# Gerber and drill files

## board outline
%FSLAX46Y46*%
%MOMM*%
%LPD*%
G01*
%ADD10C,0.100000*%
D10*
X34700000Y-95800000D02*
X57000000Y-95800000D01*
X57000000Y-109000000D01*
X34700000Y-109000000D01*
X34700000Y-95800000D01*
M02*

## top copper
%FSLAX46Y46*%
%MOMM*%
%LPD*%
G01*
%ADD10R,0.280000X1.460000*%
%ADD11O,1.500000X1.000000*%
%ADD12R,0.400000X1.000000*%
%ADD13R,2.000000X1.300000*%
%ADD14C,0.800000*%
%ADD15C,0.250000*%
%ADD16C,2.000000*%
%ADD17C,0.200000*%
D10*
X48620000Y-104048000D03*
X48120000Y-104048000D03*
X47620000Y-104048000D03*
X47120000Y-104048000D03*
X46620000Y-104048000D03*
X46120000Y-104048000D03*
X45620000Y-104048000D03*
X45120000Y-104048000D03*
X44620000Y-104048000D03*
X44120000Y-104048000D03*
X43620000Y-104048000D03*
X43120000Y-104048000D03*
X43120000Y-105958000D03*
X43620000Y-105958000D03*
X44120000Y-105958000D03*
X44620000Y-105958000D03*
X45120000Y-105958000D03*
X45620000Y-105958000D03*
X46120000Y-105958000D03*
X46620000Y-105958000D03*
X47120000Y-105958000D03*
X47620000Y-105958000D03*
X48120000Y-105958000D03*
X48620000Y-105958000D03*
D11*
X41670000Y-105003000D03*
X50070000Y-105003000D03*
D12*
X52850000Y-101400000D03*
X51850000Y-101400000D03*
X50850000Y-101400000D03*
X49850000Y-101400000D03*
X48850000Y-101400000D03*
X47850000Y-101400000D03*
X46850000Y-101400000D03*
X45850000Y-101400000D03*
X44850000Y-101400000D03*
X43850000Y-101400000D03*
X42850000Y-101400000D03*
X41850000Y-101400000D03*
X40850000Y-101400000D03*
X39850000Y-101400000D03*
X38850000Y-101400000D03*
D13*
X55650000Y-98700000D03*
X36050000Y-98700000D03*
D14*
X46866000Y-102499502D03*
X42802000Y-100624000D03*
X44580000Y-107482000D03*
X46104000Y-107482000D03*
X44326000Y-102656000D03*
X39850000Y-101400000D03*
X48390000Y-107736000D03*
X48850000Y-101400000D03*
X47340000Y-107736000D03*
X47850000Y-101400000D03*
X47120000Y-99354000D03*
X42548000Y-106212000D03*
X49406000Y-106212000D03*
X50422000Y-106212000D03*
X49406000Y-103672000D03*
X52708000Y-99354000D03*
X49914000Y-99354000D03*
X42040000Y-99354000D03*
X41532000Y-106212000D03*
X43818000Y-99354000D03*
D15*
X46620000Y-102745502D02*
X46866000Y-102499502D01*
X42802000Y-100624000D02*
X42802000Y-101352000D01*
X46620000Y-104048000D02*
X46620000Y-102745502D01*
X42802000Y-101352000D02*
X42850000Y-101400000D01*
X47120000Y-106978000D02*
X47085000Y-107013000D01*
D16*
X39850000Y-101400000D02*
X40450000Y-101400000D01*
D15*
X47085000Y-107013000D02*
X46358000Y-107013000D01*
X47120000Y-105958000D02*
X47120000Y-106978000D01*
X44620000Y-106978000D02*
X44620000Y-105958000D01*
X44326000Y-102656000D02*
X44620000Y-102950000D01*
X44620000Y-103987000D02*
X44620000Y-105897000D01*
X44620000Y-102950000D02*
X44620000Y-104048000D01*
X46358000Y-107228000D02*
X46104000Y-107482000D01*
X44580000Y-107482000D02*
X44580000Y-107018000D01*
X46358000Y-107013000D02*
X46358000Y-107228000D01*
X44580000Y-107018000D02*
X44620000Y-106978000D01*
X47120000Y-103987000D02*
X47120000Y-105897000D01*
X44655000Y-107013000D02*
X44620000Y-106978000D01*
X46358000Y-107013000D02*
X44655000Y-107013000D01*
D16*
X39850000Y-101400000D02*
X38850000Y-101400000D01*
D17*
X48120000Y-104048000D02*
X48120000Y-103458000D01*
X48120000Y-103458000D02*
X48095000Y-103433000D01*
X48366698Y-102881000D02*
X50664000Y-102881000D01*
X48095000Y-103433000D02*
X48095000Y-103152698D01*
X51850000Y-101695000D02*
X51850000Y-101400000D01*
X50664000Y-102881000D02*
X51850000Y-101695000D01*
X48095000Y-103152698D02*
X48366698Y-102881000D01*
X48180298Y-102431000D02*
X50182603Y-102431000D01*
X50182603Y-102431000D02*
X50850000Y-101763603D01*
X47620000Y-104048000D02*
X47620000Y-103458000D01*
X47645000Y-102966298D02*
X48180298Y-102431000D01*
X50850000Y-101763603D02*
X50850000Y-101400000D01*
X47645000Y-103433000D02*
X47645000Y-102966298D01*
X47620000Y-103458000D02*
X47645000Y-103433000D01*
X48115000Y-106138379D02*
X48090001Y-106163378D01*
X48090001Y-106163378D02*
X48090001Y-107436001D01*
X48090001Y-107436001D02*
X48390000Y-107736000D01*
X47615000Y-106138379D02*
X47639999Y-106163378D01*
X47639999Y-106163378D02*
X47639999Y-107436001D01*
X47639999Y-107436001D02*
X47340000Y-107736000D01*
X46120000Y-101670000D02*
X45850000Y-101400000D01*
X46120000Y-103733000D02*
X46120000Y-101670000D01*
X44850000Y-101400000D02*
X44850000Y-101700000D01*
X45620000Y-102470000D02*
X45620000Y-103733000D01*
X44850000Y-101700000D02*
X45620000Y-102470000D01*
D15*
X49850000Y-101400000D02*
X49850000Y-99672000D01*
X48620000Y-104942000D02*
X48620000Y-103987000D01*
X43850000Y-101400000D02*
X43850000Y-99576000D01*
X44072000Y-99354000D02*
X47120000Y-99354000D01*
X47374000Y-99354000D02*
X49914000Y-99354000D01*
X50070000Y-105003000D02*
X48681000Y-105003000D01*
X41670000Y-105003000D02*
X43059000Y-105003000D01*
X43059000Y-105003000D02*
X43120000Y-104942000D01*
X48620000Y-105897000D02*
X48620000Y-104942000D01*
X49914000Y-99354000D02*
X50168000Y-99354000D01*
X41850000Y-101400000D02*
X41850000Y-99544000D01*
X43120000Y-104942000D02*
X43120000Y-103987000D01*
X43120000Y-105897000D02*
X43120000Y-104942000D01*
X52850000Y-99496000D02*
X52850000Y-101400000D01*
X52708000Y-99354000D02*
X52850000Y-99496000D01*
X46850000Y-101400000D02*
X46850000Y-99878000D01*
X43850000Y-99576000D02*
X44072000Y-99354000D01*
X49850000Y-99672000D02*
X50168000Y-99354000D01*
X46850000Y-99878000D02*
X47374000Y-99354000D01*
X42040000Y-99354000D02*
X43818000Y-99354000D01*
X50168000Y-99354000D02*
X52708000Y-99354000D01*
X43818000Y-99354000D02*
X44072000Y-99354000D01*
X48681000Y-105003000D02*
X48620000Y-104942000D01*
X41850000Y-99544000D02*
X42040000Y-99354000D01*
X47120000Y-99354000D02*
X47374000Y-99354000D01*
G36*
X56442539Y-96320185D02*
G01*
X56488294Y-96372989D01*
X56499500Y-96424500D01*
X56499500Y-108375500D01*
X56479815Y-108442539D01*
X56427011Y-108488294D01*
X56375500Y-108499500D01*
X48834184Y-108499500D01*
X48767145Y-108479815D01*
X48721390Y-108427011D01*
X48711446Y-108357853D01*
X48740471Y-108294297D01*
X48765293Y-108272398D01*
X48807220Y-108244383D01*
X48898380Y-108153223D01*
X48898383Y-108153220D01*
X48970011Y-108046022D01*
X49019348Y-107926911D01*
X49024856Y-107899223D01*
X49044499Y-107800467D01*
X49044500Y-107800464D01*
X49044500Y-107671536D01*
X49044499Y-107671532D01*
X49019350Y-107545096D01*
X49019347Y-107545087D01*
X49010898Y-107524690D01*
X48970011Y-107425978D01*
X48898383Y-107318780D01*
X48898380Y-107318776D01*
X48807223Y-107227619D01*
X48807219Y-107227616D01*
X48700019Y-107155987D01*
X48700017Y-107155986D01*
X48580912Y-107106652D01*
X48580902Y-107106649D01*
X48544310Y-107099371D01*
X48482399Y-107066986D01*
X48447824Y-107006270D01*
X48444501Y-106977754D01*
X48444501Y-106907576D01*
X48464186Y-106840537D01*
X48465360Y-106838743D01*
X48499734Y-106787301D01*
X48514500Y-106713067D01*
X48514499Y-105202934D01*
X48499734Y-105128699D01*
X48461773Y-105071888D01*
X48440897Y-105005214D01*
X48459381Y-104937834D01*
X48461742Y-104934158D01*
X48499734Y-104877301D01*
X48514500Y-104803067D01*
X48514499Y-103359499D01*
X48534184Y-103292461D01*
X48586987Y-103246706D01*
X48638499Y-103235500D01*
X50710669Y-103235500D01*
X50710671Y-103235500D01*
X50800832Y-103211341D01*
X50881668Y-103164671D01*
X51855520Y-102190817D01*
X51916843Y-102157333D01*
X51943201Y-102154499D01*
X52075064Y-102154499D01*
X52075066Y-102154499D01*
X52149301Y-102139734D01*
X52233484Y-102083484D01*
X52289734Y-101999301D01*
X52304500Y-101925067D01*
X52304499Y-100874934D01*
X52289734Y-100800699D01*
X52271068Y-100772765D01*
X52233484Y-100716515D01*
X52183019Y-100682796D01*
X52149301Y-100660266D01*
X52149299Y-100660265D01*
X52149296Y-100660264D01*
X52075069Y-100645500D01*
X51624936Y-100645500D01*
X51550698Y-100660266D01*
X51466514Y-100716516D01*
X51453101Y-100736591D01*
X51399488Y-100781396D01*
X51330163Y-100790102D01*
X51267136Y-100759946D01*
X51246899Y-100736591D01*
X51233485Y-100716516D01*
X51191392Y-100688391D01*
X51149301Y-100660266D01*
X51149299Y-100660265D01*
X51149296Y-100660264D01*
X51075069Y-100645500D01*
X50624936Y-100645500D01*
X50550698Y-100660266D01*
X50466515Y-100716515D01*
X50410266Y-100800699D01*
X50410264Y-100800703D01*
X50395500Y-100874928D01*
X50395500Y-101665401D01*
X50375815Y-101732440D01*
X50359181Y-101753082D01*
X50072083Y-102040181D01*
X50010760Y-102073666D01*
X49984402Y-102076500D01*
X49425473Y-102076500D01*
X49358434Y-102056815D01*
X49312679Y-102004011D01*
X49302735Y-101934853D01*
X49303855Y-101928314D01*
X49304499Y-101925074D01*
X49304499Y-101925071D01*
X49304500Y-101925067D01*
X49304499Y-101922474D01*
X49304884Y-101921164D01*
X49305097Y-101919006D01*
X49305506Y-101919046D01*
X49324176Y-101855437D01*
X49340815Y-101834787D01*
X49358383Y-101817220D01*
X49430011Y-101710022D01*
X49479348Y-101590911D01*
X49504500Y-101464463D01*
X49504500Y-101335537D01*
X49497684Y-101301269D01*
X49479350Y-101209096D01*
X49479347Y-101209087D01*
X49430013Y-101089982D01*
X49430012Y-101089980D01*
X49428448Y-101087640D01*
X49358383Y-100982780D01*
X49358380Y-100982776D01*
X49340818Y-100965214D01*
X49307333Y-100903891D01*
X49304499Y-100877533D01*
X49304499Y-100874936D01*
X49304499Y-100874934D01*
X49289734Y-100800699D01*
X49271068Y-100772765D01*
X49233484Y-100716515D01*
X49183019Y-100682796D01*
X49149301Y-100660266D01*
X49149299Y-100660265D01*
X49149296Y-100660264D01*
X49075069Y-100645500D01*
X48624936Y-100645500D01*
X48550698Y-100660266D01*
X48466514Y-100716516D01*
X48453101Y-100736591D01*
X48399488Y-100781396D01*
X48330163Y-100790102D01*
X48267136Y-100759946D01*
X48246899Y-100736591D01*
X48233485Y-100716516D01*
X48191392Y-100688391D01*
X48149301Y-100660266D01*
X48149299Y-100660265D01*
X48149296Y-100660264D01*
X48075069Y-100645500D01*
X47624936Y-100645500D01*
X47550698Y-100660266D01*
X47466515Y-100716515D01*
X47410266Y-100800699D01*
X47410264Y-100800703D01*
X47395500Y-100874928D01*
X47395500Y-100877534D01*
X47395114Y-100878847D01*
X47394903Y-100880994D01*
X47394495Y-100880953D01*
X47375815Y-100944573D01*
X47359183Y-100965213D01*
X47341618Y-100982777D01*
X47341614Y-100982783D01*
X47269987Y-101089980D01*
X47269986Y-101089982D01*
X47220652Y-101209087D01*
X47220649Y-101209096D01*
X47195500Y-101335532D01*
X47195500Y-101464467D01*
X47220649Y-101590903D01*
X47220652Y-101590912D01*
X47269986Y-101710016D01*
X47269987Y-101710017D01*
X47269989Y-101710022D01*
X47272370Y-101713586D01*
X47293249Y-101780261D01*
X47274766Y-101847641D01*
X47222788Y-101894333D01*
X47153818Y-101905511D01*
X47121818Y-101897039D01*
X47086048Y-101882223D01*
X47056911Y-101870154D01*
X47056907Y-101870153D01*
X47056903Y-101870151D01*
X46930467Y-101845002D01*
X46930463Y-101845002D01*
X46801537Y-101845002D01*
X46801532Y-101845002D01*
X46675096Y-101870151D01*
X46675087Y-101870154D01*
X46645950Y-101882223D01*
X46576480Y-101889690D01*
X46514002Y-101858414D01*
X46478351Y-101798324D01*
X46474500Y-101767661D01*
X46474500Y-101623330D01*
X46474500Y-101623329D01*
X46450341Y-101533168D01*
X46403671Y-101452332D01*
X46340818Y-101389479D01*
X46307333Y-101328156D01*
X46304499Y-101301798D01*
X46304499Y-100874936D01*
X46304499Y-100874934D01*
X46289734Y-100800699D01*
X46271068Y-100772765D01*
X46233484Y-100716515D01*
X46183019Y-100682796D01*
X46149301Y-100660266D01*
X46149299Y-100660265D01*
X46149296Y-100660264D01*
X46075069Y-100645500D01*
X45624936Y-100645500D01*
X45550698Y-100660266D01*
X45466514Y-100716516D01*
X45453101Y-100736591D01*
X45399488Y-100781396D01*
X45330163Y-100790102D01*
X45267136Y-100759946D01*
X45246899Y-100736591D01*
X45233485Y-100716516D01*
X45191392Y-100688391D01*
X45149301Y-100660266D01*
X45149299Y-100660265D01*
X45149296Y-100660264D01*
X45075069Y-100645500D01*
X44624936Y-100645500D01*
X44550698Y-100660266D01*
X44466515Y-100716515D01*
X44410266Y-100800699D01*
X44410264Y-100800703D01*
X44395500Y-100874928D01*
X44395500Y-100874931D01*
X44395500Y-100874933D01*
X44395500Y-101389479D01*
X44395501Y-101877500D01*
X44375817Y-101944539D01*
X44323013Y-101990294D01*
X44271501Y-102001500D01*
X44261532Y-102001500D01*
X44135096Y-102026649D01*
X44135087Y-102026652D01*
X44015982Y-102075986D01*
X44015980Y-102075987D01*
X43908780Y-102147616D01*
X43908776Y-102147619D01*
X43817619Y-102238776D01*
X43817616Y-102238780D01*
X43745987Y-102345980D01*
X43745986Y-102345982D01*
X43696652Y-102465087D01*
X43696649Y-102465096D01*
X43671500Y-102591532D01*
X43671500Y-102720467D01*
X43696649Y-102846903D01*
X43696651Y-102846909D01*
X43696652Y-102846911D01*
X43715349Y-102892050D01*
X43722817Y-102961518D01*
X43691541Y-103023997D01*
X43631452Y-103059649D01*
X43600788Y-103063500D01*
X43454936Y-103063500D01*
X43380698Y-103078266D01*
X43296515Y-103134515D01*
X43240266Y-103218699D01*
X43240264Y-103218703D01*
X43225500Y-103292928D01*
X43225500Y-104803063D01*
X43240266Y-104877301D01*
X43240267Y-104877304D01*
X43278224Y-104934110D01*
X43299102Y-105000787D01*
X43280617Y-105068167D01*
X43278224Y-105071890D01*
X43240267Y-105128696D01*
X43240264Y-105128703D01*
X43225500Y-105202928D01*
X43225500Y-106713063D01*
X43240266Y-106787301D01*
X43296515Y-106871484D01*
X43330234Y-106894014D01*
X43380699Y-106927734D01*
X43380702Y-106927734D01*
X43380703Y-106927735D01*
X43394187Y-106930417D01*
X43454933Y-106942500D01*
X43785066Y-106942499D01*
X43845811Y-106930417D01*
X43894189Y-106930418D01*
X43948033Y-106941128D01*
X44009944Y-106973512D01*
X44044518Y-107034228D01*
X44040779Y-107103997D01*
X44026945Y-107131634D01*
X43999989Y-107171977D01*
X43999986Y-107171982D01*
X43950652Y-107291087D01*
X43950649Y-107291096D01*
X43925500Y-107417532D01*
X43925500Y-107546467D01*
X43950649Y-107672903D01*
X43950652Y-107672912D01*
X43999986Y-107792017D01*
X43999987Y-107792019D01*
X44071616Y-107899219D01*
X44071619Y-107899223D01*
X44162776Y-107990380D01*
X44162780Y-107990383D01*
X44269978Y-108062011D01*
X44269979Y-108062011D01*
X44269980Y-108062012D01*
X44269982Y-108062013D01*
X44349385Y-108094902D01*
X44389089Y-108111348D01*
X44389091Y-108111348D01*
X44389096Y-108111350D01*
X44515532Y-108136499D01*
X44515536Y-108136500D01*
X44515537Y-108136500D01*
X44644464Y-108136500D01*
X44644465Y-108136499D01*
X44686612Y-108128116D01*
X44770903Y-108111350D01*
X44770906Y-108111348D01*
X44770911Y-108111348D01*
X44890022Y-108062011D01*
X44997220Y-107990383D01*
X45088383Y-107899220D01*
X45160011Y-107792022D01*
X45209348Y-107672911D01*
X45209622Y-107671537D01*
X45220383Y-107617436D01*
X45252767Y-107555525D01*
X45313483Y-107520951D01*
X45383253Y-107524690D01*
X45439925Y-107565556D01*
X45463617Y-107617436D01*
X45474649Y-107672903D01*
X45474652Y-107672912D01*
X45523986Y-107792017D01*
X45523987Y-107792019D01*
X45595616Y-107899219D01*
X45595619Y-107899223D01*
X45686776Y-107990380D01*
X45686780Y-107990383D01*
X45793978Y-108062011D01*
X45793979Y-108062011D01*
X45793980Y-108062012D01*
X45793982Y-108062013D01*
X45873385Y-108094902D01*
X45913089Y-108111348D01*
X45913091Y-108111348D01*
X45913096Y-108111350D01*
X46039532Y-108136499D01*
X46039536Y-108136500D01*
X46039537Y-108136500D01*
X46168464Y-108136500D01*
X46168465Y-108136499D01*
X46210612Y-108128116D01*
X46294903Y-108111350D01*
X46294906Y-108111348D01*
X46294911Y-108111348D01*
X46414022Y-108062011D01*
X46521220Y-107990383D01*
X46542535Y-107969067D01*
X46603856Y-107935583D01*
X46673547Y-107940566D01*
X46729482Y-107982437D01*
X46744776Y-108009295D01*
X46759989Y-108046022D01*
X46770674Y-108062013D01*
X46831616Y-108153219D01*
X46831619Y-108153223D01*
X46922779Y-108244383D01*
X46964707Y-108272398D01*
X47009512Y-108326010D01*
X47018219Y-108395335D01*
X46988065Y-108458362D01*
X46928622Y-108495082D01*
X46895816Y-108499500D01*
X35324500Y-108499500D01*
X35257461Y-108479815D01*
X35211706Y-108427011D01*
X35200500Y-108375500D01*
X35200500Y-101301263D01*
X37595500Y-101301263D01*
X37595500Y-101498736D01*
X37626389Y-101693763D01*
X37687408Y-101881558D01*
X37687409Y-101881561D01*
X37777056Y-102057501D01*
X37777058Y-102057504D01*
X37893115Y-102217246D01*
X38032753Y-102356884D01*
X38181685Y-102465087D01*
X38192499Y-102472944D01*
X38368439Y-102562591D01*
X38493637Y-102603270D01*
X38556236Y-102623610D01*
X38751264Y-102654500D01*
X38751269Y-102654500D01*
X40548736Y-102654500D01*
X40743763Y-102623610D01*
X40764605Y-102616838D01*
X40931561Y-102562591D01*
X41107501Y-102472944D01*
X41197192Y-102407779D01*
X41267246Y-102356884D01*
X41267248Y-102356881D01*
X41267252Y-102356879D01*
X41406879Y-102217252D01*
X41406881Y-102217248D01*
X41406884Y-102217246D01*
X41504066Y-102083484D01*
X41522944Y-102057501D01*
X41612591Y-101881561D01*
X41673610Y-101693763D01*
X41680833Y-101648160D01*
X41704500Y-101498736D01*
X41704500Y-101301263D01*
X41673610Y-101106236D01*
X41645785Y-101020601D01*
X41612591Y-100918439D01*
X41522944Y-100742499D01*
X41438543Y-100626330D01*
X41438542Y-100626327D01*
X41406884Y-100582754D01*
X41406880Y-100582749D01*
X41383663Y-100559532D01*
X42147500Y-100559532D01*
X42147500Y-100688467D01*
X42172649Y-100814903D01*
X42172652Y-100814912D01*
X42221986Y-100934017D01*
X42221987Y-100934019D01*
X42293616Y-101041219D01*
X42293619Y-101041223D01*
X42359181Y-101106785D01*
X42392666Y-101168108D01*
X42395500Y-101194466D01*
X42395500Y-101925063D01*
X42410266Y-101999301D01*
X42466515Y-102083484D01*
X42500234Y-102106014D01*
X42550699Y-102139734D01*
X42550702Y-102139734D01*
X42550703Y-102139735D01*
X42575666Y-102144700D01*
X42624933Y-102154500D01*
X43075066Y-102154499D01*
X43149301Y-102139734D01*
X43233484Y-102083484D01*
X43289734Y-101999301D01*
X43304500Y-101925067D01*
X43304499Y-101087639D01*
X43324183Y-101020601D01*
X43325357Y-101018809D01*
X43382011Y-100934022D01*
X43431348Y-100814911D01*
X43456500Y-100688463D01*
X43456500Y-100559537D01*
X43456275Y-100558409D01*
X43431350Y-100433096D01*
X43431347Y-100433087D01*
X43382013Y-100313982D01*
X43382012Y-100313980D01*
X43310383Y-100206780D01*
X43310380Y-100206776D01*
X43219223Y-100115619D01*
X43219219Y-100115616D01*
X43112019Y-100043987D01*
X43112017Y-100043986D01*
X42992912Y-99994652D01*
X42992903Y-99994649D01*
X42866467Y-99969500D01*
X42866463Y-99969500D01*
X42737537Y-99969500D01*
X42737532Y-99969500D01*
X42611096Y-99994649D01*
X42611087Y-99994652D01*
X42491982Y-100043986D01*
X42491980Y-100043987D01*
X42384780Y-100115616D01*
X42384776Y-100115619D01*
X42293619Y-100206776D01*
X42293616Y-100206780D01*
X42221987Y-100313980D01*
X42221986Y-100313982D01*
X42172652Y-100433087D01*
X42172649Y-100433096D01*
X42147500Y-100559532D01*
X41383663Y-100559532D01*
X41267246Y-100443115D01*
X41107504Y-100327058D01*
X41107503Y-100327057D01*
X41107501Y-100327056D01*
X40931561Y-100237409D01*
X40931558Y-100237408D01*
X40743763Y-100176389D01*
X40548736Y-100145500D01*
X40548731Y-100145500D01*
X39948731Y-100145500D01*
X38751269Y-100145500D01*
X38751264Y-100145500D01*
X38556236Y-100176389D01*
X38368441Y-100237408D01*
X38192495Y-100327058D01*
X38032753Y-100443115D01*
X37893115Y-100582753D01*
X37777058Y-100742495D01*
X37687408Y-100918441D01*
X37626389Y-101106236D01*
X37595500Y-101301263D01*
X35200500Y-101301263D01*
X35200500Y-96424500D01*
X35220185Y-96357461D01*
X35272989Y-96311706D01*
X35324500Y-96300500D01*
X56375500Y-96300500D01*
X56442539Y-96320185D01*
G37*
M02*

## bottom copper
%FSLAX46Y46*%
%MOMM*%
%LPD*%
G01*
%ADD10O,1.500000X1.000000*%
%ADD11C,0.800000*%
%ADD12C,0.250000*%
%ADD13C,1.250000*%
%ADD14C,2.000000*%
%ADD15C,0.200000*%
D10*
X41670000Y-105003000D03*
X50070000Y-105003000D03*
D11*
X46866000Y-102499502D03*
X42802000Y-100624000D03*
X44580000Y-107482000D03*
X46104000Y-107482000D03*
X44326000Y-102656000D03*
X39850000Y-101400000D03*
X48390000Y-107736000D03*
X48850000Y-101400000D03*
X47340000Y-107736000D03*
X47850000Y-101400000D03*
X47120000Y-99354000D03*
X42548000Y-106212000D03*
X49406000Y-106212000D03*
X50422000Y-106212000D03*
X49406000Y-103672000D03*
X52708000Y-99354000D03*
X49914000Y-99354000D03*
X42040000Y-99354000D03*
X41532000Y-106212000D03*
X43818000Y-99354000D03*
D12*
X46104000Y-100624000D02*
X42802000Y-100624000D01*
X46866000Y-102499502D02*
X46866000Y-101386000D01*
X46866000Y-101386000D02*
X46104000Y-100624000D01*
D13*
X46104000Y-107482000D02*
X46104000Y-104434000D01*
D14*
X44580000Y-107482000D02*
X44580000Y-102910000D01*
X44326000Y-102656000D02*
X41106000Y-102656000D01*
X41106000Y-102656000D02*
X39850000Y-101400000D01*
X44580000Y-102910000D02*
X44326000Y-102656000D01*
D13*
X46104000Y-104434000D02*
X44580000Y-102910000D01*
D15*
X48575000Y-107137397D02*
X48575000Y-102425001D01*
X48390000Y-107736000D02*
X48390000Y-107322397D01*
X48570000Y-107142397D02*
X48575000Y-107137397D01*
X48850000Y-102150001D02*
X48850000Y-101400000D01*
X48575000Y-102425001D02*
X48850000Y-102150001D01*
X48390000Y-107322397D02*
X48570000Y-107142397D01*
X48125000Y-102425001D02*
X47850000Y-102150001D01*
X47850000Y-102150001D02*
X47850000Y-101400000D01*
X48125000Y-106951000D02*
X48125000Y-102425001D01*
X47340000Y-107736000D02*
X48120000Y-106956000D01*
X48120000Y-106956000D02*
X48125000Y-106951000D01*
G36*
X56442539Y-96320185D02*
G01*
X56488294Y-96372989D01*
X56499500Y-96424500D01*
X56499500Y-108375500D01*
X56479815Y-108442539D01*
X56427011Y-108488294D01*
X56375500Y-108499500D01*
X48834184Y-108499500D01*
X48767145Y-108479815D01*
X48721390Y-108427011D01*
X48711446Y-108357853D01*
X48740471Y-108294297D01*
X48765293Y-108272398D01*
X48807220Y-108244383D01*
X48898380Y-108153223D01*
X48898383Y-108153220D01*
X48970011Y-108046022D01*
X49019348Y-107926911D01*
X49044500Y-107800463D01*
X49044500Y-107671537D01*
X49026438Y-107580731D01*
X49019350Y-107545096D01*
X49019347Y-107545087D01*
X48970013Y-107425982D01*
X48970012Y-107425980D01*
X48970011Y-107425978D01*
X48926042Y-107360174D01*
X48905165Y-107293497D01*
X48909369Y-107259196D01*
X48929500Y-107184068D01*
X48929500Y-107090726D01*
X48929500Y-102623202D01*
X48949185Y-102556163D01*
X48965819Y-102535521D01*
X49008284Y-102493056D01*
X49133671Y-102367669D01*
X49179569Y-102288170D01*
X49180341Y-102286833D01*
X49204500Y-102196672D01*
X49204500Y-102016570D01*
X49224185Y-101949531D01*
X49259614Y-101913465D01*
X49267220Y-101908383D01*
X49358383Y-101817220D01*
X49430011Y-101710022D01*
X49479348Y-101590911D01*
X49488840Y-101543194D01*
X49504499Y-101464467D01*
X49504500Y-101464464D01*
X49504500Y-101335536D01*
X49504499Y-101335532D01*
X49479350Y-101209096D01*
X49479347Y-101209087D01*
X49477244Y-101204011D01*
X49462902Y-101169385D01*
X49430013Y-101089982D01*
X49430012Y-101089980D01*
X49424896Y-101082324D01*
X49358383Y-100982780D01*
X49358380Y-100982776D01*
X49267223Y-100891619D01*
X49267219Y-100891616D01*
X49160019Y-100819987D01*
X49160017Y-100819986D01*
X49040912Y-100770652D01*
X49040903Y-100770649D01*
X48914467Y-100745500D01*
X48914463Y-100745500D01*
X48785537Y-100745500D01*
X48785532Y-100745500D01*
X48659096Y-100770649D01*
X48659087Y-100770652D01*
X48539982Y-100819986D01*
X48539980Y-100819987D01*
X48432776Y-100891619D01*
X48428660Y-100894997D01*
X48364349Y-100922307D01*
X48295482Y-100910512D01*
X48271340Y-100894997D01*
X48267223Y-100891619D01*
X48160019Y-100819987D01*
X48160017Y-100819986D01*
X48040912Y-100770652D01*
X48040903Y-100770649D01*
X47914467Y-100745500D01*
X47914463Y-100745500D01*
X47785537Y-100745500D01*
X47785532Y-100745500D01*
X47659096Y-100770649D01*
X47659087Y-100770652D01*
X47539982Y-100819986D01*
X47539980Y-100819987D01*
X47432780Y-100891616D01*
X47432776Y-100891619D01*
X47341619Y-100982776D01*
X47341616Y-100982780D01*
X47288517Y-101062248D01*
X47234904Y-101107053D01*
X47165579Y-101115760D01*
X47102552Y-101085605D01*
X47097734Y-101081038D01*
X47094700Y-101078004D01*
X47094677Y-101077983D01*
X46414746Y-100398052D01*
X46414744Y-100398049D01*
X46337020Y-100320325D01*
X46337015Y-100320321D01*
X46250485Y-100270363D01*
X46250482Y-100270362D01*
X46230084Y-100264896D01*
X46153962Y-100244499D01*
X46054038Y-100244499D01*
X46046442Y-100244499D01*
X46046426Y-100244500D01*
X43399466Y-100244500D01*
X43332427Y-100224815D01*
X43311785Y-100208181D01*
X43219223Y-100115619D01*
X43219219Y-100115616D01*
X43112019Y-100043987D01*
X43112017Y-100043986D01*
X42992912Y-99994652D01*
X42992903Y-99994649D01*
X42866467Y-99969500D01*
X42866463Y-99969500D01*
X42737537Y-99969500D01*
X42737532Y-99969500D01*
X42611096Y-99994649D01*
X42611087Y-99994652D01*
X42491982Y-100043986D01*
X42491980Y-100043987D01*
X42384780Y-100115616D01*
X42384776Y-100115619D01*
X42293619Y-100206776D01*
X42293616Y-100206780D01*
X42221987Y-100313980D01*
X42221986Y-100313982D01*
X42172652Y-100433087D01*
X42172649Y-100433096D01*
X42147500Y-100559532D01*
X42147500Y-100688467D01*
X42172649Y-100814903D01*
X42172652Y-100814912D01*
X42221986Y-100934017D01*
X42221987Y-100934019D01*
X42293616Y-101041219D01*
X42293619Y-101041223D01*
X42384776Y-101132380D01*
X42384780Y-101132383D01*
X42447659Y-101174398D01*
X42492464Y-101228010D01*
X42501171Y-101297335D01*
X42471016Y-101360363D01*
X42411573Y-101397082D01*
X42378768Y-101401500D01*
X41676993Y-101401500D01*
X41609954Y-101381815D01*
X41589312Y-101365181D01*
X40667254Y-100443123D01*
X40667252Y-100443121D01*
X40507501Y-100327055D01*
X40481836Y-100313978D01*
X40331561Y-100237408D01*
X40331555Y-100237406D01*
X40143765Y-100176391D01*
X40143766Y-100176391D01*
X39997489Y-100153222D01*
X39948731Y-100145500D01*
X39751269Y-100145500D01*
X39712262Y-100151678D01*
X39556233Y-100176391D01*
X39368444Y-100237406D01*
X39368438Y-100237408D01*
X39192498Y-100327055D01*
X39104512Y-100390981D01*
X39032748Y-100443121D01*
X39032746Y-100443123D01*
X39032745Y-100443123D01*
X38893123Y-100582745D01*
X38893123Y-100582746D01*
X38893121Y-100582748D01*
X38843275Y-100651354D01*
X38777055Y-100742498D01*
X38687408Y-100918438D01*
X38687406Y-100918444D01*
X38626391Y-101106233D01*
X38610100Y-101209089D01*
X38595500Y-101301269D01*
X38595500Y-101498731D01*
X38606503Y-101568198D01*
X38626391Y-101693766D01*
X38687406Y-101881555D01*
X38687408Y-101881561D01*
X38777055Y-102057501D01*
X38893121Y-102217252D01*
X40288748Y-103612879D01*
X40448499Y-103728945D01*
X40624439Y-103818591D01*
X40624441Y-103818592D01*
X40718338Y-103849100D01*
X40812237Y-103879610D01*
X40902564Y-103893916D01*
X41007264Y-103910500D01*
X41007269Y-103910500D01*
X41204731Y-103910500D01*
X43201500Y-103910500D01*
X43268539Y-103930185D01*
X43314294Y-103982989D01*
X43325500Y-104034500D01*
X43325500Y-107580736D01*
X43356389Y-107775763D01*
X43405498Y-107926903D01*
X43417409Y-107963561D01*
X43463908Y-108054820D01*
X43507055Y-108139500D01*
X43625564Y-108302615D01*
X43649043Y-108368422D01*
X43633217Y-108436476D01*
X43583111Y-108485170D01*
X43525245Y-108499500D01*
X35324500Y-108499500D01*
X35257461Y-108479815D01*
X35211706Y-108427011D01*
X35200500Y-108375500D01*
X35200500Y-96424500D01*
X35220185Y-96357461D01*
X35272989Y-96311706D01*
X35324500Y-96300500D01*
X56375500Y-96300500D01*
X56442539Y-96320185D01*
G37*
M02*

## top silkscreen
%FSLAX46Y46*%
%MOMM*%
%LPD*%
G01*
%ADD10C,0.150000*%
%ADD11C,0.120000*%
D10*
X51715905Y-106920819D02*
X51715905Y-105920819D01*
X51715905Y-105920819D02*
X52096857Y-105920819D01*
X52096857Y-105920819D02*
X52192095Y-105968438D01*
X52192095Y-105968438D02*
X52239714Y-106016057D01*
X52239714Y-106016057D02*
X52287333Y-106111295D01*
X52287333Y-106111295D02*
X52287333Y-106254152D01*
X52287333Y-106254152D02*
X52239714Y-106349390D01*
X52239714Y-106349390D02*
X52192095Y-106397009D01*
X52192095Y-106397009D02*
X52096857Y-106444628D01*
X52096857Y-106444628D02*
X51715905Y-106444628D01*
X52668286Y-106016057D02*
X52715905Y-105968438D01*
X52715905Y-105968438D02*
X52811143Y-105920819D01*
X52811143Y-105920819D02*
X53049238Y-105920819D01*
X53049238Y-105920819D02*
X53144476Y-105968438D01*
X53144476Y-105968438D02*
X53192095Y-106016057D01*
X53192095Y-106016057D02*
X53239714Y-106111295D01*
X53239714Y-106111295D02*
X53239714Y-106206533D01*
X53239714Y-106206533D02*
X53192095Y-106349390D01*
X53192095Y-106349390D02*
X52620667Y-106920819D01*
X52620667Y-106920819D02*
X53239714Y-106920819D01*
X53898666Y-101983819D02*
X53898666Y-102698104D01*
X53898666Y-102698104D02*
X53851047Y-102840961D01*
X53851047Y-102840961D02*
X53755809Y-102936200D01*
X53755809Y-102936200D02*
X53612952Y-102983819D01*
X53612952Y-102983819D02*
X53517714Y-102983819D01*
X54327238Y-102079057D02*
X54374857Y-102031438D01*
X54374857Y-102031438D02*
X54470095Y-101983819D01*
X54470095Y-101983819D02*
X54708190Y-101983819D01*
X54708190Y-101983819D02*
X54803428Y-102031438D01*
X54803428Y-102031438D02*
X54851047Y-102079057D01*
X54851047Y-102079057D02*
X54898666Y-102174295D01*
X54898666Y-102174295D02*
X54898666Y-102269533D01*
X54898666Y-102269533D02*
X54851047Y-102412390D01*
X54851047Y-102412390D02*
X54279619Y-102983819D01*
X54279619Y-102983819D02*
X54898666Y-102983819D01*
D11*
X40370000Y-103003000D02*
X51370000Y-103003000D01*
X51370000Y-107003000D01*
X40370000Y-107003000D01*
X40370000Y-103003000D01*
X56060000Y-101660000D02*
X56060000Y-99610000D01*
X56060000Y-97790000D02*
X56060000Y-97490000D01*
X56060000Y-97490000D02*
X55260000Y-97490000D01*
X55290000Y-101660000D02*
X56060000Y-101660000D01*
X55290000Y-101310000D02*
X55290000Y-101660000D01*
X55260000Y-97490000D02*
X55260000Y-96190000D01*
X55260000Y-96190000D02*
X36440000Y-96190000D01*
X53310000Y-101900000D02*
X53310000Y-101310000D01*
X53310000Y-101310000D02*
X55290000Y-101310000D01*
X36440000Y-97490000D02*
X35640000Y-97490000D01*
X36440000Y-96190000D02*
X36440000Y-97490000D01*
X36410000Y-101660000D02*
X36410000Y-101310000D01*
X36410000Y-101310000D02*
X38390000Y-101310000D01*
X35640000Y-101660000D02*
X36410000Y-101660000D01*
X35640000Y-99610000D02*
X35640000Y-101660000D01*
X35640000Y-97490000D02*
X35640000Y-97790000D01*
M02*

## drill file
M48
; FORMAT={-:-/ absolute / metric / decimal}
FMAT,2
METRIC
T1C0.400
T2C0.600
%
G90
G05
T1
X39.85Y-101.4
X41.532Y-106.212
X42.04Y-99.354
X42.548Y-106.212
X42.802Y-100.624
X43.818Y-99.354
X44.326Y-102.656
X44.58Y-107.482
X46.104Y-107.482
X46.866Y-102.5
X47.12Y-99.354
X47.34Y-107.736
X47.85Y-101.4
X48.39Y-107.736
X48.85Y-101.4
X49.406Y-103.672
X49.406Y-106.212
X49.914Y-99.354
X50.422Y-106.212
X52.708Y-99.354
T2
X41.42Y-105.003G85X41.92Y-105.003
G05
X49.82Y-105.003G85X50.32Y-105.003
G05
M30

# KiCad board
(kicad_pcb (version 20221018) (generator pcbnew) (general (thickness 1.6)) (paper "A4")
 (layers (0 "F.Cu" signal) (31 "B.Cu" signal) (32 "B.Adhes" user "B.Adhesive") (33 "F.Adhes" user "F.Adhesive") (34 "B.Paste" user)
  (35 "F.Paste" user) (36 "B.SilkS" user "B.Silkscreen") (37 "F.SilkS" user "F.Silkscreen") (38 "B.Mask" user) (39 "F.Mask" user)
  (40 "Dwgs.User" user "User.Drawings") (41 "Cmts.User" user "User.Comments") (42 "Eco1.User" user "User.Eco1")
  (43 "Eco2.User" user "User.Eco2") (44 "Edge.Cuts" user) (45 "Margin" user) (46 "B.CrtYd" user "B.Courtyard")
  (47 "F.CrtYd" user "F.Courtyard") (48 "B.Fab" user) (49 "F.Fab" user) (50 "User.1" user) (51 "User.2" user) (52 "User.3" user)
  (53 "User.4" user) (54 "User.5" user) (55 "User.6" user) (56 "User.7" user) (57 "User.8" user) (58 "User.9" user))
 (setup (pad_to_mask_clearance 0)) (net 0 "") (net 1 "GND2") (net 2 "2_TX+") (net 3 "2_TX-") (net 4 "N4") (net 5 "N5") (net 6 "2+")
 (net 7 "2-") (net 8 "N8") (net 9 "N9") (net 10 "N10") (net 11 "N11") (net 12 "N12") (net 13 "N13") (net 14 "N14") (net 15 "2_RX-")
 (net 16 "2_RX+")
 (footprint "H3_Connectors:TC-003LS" (layer "F.Cu") (at 45.87 105.003)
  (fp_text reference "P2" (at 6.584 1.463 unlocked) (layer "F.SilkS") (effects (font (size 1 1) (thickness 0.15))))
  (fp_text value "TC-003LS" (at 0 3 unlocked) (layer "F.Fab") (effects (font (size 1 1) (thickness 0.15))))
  (fp_rect (start -5.5 -2) (end 5.5 2) (stroke (width 0.12) (type default)) (fill none) (layer "F.SilkS"))
  (pad "A1" smd rect (at 2.75 -0.955) (size 0.28 1.46) (layers "F.Cu" "F.Paste" "F.Mask") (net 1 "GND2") (thermal_bridge_angle 45))
  (pad "A2" smd rect (at 2.25 -0.955) (size 0.28 1.46) (layers "F.Cu" "F.Paste" "F.Mask") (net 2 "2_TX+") (thermal_bridge_angle 45))
  (pad "A3" smd rect (at 1.75 -0.955) (size 0.28 1.46) (layers "F.Cu" "F.Paste" "F.Mask") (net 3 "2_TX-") (thermal_bridge_angle 45))
  (pad "A4" smd rect (at 1.25 -0.955) (size 0.28 1.46) (layers "F.Cu" "F.Paste" "F.Mask") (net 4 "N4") (thermal_bridge_angle 45))
  (pad "A5" smd rect (at 0.75 -0.955) (size 0.28 1.46) (layers "F.Cu" "F.Paste" "F.Mask") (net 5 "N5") (thermal_bridge_angle 45))
  (pad "A6" smd rect (at 0.25 -0.955) (size 0.28 1.46) (layers "F.Cu" "F.Paste" "F.Mask") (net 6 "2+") (thermal_bridge_angle 45))
  (pad "A7" smd rect (at -0.25 -0.955) (size 0.28 1.46) (layers "F.Cu" "F.Paste" "F.Mask") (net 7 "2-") (thermal_bridge_angle 45))
  (pad "A8" smd rect (at -0.75 -0.955) (size 0.28 1.46) (layers "F.Cu" "F.Paste" "F.Mask") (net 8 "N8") (thermal_bridge_angle 45))
  (pad "A9" smd rect (at -1.25 -0.955) (size 0.28 1.46) (layers "F.Cu" "F.Paste" "F.Mask") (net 4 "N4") (thermal_bridge_angle 45))
  (pad "A10" smd rect (at -1.75 -0.955) (size 0.28 1.46) (layers "F.Cu" "F.Paste" "F.Mask") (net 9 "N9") (thermal_bridge_angle 45))
  (pad "A11" smd rect (at -2.25 -0.955) (size 0.28 1.46) (layers "F.Cu" "F.Paste" "F.Mask") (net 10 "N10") (thermal_bridge_angle 45))
  (pad "A12" smd rect (at -2.75 -0.955) (size 0.28 1.46) (layers "F.Cu" "F.Paste" "F.Mask") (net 1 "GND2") (thermal_bridge_angle 45))
  (pad "B1" smd rect (at -2.75 0.955 180) (size 0.28 1.46) (layers "F.Cu" "F.Paste" "F.Mask") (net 1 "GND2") (thermal_bridge_angle 45))
  (pad "B2" smd rect (at -2.25 0.955 180) (size 0.28 1.46) (layers "F.Cu" "F.Paste" "F.Mask") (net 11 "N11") (thermal_bridge_angle 45))
  (pad "B3" smd rect (at -1.75 0.955 180) (size 0.28 1.46) (layers "F.Cu" "F.Paste" "F.Mask") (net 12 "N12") (thermal_bridge_angle 45))
  (pad "B4" smd rect (at -1.25 0.955 180) (size 0.28 1.46) (layers "F.Cu" "F.Paste" "F.Mask") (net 4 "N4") (thermal_bridge_angle 45))
  (pad "B5" smd rect (at -0.75 0.955 180) (size 0.28 1.46) (layers "F.Cu" "F.Paste" "F.Mask") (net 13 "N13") (thermal_bridge_angle 45))
  (pad "B6" smd rect (at -0.25 0.955 180) (size 0.28 1.46) (layers "F.Cu" "F.Paste" "F.Mask") (thermal_bridge_angle 45))
  (pad "B7" smd rect (at 0.25 0.955 180) (size 0.28 1.46) (layers "F.Cu" "F.Paste" "F.Mask") (thermal_bridge_angle 45))
  (pad "B8" smd rect (at 0.75 0.955 180) (size 0.28 1.46) (layers "F.Cu" "F.Paste" "F.Mask") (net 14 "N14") (thermal_bridge_angle 45))
  (pad "B9" smd rect (at 1.25 0.955 180) (size 0.28 1.46) (layers "F.Cu" "F.Paste" "F.Mask") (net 4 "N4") (thermal_bridge_angle 45))
  (pad "B10" smd rect (at 1.75 0.955 180) (size 0.28 1.46) (layers "F.Cu" "F.Paste" "F.Mask") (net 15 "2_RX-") (thermal_bridge_angle 45))
  (pad "B11" smd rect (at 2.25 0.955 180) (size 0.28 1.46) (layers "F.Cu" "F.Paste" "F.Mask") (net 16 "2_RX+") (thermal_bridge_angle 45))
  (pad "B12" smd rect (at 2.75 0.955 180) (size 0.28 1.46) (layers "F.Cu" "F.Paste" "F.Mask") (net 1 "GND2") (thermal_bridge_angle 45))
  (pad "S1" thru_hole oval (at -4.2 0) (size 1.5 1) (drill oval 1.1 0.6) (layers "*.Cu" "*.Mask") (remove_unused_layers) (keep_end_layers)
   (zone_layer_connections) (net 1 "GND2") (thermal_bridge_angle 45))
  (pad "S1" thru_hole oval (at 4.2 0) (size 1.5 1) (drill oval 1.1 0.6) (layers "*.Cu" "*.Mask") (remove_unused_layers) (keep_end_layers)
   (zone_layer_connections) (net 1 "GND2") (thermal_bridge_angle 45)))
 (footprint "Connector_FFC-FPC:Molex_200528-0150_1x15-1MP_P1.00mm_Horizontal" (layer "F.Cu") (at 45.85 100.49 180)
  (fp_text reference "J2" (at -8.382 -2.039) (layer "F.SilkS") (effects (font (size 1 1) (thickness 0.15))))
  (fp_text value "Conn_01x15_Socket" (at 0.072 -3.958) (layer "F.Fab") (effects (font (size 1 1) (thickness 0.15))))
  (fp_line (start -10.21 -1.17) (end -10.21 0.88) (stroke (width 0.12) (type solid)) (layer "F.SilkS"))
  (fp_line (start -10.21 2.7) (end -10.21 3) (stroke (width 0.12) (type solid)) (layer "F.SilkS"))
  (fp_line (start -10.21 3) (end -9.41 3) (stroke (width 0.12) (type solid)) (layer "F.SilkS"))
  (fp_line (start -9.44 -1.17) (end -10.21 -1.17) (stroke (width 0.12) (type solid)) (layer "F.SilkS"))
  (fp_line (start -9.44 -0.82) (end -9.44 -1.17) (stroke (width 0.12) (type solid)) (layer "F.SilkS"))
  (fp_line (start -9.41 3) (end -9.41 4.3) (stroke (width 0.12) (type solid)) (layer "F.SilkS"))
  (fp_line (start -9.41 4.3) (end 9.41 4.3) (stroke (width 0.12) (type solid)) (layer "F.SilkS"))
  (fp_line (start -7.46 -1.41) (end -7.46 -0.82) (stroke (width 0.12) (type solid)) (layer "F.SilkS"))
  (fp_line (start -7.46 -0.82) (end -9.44 -0.82) (stroke (width 0.12) (type solid)) (layer "F.SilkS"))
  (fp_line (start 9.41 3) (end 10.21 3) (stroke (width 0.12) (type solid)) (layer "F.SilkS"))
  (fp_line (start 9.41 4.3) (end 9.41 3) (stroke (width 0.12) (type solid)) (layer "F.SilkS"))
  (fp_line (start 9.44 -1.17) (end 9.44 -0.82) (stroke (width 0.12) (type solid)) (layer "F.SilkS"))
  (fp_line (start 9.44 -0.82) (end 7.46 -0.82) (stroke (width 0.12) (type solid)) (layer "F.SilkS"))
  (fp_line (start 10.21 -1.17) (end 9.44 -1.17) (stroke (width 0.12) (type solid)) (layer "F.SilkS"))
  (fp_line (start 10.21 0.88) (end 10.21 -1.17) (stroke (width 0.12) (type solid)) (layer "F.SilkS"))
  (fp_line (start 10.21 3) (end 10.21 2.7) (stroke (width 0.12) (type solid)) (layer "F.SilkS"))
  (pad "1" smd rect (at -7 -0.91 180) (size 0.4 1) (layers "F.Cu" "F.Paste" "F.Mask") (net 1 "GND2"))
  (pad "2" smd rect (at -6 -0.91 180) (size 0.4 1) (layers "F.Cu" "F.Paste" "F.Mask") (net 2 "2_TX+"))
  (pad "3" smd rect (at -5 -0.91 180) (size 0.4 1) (layers "F.Cu" "F.Paste" "F.Mask") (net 3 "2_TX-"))
  (pad "4" smd rect (at -4 -0.91 180) (size 0.4 1) (layers "F.Cu" "F.Paste" "F.Mask") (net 1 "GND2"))
  (pad "5" smd rect (at -3 -0.91 180) (size 0.4 1) (layers "F.Cu" "F.Paste" "F.Mask") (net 16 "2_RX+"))
  (pad "6" smd rect (at -2 -0.91 180) (size 0.4 1) (layers "F.Cu" "F.Paste" "F.Mask") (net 15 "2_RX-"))
  (pad "7" smd rect (at -1 -0.91 180) (size 0.4 1) (layers "F.Cu" "F.Paste" "F.Mask") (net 1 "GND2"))
  (pad "8" smd rect (at 0 -0.91 180) (size 0.4 1) (layers "F.Cu" "F.Paste" "F.Mask") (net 6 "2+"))
  (pad "9" smd rect (at 1 -0.91 180) (size 0.4 1) (layers "F.Cu" "F.Paste" "F.Mask") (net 7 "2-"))
  (pad "10" smd rect (at 2 -0.91 180) (size 0.4 1) (layers "F.Cu" "F.Paste" "F.Mask") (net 1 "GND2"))
  (pad "11" smd rect (at 3 -0.91 180) (size 0.4 1) (layers "F.Cu" "F.Paste" "F.Mask") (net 5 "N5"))
  (pad "12" smd rect (at 4 -0.91 180) (size 0.4 1) (layers "F.Cu" "F.Paste" "F.Mask") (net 1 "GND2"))
  (pad "13" smd rect (at 5 -0.91 180) (size 0.4 1) (layers "F.Cu" "F.Paste" "F.Mask") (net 4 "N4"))
  (pad "14" smd rect (at 6 -0.91 180) (size 0.4 1) (layers "F.Cu" "F.Paste" "F.Mask") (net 4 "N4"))
  (pad "15" smd rect (at 7 -0.91 180) (size 0.4 1) (layers "F.Cu" "F.Paste" "F.Mask") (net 4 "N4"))
  (pad "MP" smd rect (at -9.8 1.79 180) (size 2 1.3) (layers "F.Cu" "F.Paste" "F.Mask") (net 1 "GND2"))
  (pad "MP" smd rect (at 9.8 1.79 180) (size 2 1.3) (layers "F.Cu" "F.Paste" "F.Mask") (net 1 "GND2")))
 (gr_rect (start 34.7 95.8) (end 57 109) (stroke (width 0.1) (type default)) (fill none) (layer "Edge.Cuts"))
 (segment (start 46.62 102.745502) (end 46.866 102.499502) (width 0.25) (layer "F.Cu") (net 5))
 (segment (start 42.802 100.624) (end 42.802 101.352) (width 0.25) (layer "F.Cu") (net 5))
 (segment (start 46.62 104.048) (end 46.62 102.745502) (width 0.25) (layer "F.Cu") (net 5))
 (segment (start 42.802 101.352) (end 42.85 101.4) (width 0.25) (layer "F.Cu") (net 5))
 (via (at 46.866 102.499502) (size 0.8) (drill 0.4) (layers "F.Cu" "B.Cu") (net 5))
 (via (at 42.802 100.624) (size 0.8) (drill 0.4) (layers "F.Cu" "B.Cu") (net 5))
 (segment (start 46.104 100.624) (end 42.802 100.624) (width 0.25) (layer "B.Cu") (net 5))
 (segment (start 46.866 102.499502) (end 46.866 101.386) (width 0.25) (layer "B.Cu") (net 5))
 (segment (start 46.866 101.386) (end 46.104 100.624) (width 0.25) (layer "B.Cu") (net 5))
 (segment (start 47.12 106.978) (end 47.085 107.013) (width 0.25) (layer "F.Cu") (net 4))
 (segment (start 39.85 101.4) (end 40.45 101.4) (width 2) (layer "F.Cu") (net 4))
 (segment (start 47.085 107.013) (end 46.358 107.013) (width 0.25) (layer "F.Cu") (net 4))
 (segment (start 47.12 105.958) (end 47.12 106.978) (width 0.25) (layer "F.Cu") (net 4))
 (segment (start 44.62 106.978) (end 44.62 105.958) (width 0.25) (layer "F.Cu") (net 4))
 (segment (start 44.326 102.656) (end 44.62 102.95) (width 0.25) (layer "F.Cu") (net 4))
 (segment (start 44.62 103.987) (end 44.62 105.897) (width 0.25) (layer "F.Cu") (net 4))
 (segment (start 44.62 102.95) (end 44.62 104.048) (width 0.25) (layer "F.Cu") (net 4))
 (segment (start 46.358 107.228) (end 46.104 107.482) (width 0.25) (layer "F.Cu") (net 4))
 (segment (start 44.58 107.482) (end 44.58 107.018) (width 0.25) (layer "F.Cu") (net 4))
 (segment (start 46.358 107.013) (end 46.358 107.228) (width 0.25) (layer "F.Cu") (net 4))
 (segment (start 44.58 107.018) (end 44.62 106.978) (width 0.25) (layer "F.Cu") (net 4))
 (segment (start 47.12 103.987) (end 47.12 105.897) (width 0.25) (layer "F.Cu") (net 4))
 (segment (start 44.655 107.013) (end 44.62 106.978) (width 0.25) (layer "F.Cu") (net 4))
 (segment (start 46.358 107.013) (end 44.655 107.013) (width 0.25) (layer "F.Cu") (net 4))
 (segment (start 39.85 101.4) (end 38.85 101.4) (width 2) (layer "F.Cu") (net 4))
 (via (at 44.58 107.482) (size 0.8) (drill 0.4) (layers "F.Cu" "B.Cu") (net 4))
 (via (at 46.104 107.482) (size 0.8) (drill 0.4) (layers "F.Cu" "B.Cu") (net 4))
 (via (at 44.326 102.656) (size 0.8) (drill 0.4) (layers "F.Cu" "B.Cu") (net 4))
 (via (at 39.85 101.4) (size 0.8) (drill 0.4) (layers "F.Cu" "B.Cu") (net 4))
 (segment (start 46.104 107.482) (end 46.104 104.434) (width 1.25) (layer "B.Cu") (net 4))
 (segment (start 44.58 107.482) (end 44.58 102.91) (width 2) (layer "B.Cu") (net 4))
 (segment (start 44.326 102.656) (end 41.106 102.656) (width 2) (layer "B.Cu") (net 4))
 (segment (start 41.106 102.656) (end 39.85 101.4) (width 2) (layer "B.Cu") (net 4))
 (segment (start 44.58 102.91) (end 44.326 102.656) (width 2) (layer "B.Cu") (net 4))
 (segment (start 46.104 104.434) (end 44.58 102.91) (width 1.25) (layer "B.Cu") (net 4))
 (segment (start 48.12 104.048) (end 48.12 103.458) (width 0.2) (layer "F.Cu") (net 2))
 (segment (start 48.12 103.458) (end 48.095 103.433) (width 0.2) (layer "F.Cu") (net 2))
 (segment (start 48.366698 102.881) (end 50.664 102.881) (width 0.2) (layer "F.Cu") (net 2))
 (segment (start 48.095 103.433) (end 48.095 103.152698) (width 0.2) (layer "F.Cu") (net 2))
 (segment (start 51.85 101.695) (end 51.85 101.4) (width 0.2) (layer "F.Cu") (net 2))
 (segment (start 50.664 102.881) (end 51.85 101.695) (width 0.2) (layer "F.Cu") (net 2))
 (segment (start 48.095 103.152698) (end 48.366698 102.881) (width 0.2) (layer "F.Cu") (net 2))
 (segment (start 48.180298 102.431) (end 50.182603 102.431) (width 0.2) (layer "F.Cu") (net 3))
 (segment (start 50.182603 102.431) (end 50.85 101.763603) (width 0.2) (layer "F.Cu") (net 3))
 (segment (start 47.62 104.048) (end 47.62 103.458) (width 0.2) (layer "F.Cu") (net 3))
 (segment (start 47.645 102.966298) (end 48.180298 102.431) (width 0.2) (layer "F.Cu") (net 3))
 (segment (start 50.85 101.763603) (end 50.85 101.4) (width 0.2) (layer "F.Cu") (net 3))
 (segment (start 47.645 103.433) (end 47.645 102.966298) (width 0.2) (layer "F.Cu") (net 3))
 (segment (start 47.62 103.458) (end 47.645 103.433) (width 0.2) (layer "F.Cu") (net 3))
 (segment (start 48.115 106.138379) (end 48.090001 106.163378) (width 0.2) (layer "F.Cu") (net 16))
 (segment (start 48.090001 106.163378) (end 48.090001 107.436001) (width 0.2) (layer "F.Cu") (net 16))
 (segment (start 48.090001 107.436001) (end 48.39 107.736) (width 0.2) (layer "F.Cu") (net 16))
 (via (at 48.39 107.736) (size 0.8) (drill 0.4) (layers "F.Cu" "B.Cu") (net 16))
 (via (at 48.85 101.4) (size 0.8) (drill 0.4) (layers "F.Cu" "B.Cu") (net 16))
 (segment (start 48.575 107.137397) (end 48.575 102.425001) (width 0.2) (layer "B.Cu") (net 16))
 (segment (start 48.39 107.736) (end 48.39 107.322397) (width 0.2) (layer "B.Cu") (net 16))
 (segment (start 48.57 107.142397) (end 48.575 107.137397) (width 0.2) (layer "B.Cu") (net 16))
 (segment (start 48.85 102.150001) (end 48.85 101.4) (width 0.2) (layer "B.Cu") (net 16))
 (segment (start 48.575 102.425001) (end 48.85 102.150001) (width 0.2) (layer "B.Cu") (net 16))
 (segment (start 48.39 107.322397) (end 48.57 107.142397) (width 0.2) (layer "B.Cu") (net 16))
 (segment (start 47.615 106.138379) (end 47.639999 106.163378) (width 0.2) (layer "F.Cu") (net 15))
 (segment (start 47.639999 106.163378) (end 47.639999 107.436001) (width 0.2) (layer "F.Cu") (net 15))
 (segment (start 47.639999 107.436001) (end 47.34 107.736) (width 0.2) (layer "F.Cu") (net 15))
 (via (at 47.34 107.736) (size 0.8) (drill 0.4) (layers "F.Cu" "B.Cu") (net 15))
 (via (at 47.85 101.4) (size 0.8) (drill 0.4) (layers "F.Cu" "B.Cu") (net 15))
 (segment (start 48.125 102.425001) (end 47.85 102.150001) (width 0.2) (layer "B.Cu") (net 15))
 (segment (start 47.85 102.150001) (end 47.85 101.4) (width 0.2) (layer "B.Cu") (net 15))
 (segment (start 48.125 106.951) (end 48.125 102.425001) (width 0.2) (layer "B.Cu") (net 15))
 (segment (start 47.34 107.736) (end 48.12 106.956) (width 0.2) (layer "B.Cu") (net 15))
 (segment (start 48.12 106.956) (end 48.125 106.951) (width 0.2) (layer "B.Cu") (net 15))
 (segment (start 46.12 101.67) (end 45.85 101.4) (width 0.2) (layer "F.Cu") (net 6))
 (segment (start 46.12 103.733) (end 46.12 101.67) (width 0.2) (layer "F.Cu") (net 6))
 (segment (start 44.85 101.4) (end 44.85 101.7) (width 0.2) (layer "F.Cu") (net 7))
 (segment (start 45.62 102.47) (end 45.62 103.733) (width 0.2) (layer "F.Cu") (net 7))
 (segment (start 44.85 101.7) (end 45.62 102.47) (width 0.2) (layer "F.Cu") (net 7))
 (segment (start 49.85 101.4) (end 49.85 99.672) (width 0.25) (layer "F.Cu") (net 1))
 (segment (start 48.62 104.942) (end 48.62 103.987) (width 0.25) (layer "F.Cu") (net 1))
 (segment (start 43.85 101.4) (end 43.85 99.576) (width 0.25) (layer "F.Cu") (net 1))
 (segment (start 44.072 99.354) (end 47.12 99.354) (width 0.25) (layer "F.Cu") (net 1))
 (segment (start 47.374 99.354) (end 49.914 99.354) (width 0.25) (layer "F.Cu") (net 1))
 (segment (start 50.07 105.003) (end 48.681 105.003) (width 0.25) (layer "F.Cu") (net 1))
 (segment (start 41.67 105.003) (end 43.059 105.003) (width 0.25) (layer "F.Cu") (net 1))
 (segment (start 43.059 105.003) (end 43.12 104.942) (width 0.25) (layer "F.Cu") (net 1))
 (segment (start 48.62 105.897) (end 48.62 104.942) (width 0.25) (layer "F.Cu") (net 1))
 (segment (start 49.914 99.354) (end 50.168 99.354) (width 0.25) (layer "F.Cu") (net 1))
 (segment (start 41.85 101.4) (end 41.85 99.544) (width 0.25) (layer "F.Cu") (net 1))
 (segment (start 43.12 104.942) (end 43.12 103.987) (width 0.25) (layer "F.Cu") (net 1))
 (segment (start 43.12 105.897) (end 43.12 104.942) (width 0.25) (layer "F.Cu") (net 1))
 (segment (start 52.85 99.496) (end 52.85 101.4) (width 0.25) (layer "F.Cu") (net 1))
 (segment (start 52.708 99.354) (end 52.85 99.496) (width 0.25) (layer "F.Cu") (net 1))
 (segment (start 46.85 101.4) (end 46.85 99.878) (width 0.25) (layer "F.Cu") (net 1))
 (segment (start 43.85 99.576) (end 44.072 99.354) (width 0.25) (layer "F.Cu") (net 1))
 (segment (start 49.85 99.672) (end 50.168 99.354) (width 0.25) (layer "F.Cu") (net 1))
 (segment (start 46.85 99.878) (end 47.374 99.354) (width 0.25) (layer "F.Cu") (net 1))
 (segment (start 42.04 99.354) (end 43.818 99.354) (width 0.25) (layer "F.Cu") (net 1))
 (segment (start 50.168 99.354) (end 52.708 99.354) (width 0.25) (layer "F.Cu") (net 1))
 (segment (start 43.818 99.354) (end 44.072 99.354) (width 0.25) (layer "F.Cu") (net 1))
 (segment (start 48.681 105.003) (end 48.62 104.942) (width 0.25) (layer "F.Cu") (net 1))
 (segment (start 41.85 99.544) (end 42.04 99.354) (width 0.25) (layer "F.Cu") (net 1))
 (segment (start 47.12 99.354) (end 47.374 99.354) (width 0.25) (layer "F.Cu") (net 1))
 (via (at 47.12 99.354) (size 0.8) (drill 0.4) (layers "F.Cu" "B.Cu") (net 1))
 (via (at 42.548 106.212) (size 0.8) (drill 0.4) (layers "F.Cu" "B.Cu") (free) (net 1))
 (via (at 49.406 106.212) (size 0.8) (drill 0.4) (layers "F.Cu" "B.Cu") (free) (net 1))
 (via (at 50.422 106.212) (size 0.8) (drill 0.4) (layers "F.Cu" "B.Cu") (free) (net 1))
 (via (at 49.406 103.672) (size 0.8) (drill 0.4) (layers "F.Cu" "B.Cu") (free) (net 1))
 (via (at 52.708 99.354) (size 0.8) (drill 0.4) (layers "F.Cu" "B.Cu") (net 1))
 (via (at 49.914 99.354) (size 0.8) (drill 0.4) (layers "F.Cu" "B.Cu") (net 1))
 (via (at 42.04 99.354) (size 0.8) (drill 0.4) (layers "F.Cu" "B.Cu") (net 1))
 (via (at 41.532 106.212) (size 0.8) (drill 0.4) (layers "F.Cu" "B.Cu") (free) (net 1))
 (via (at 43.818 99.354) (size 0.8) (drill 0.4) (layers "F.Cu" "B.Cu") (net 1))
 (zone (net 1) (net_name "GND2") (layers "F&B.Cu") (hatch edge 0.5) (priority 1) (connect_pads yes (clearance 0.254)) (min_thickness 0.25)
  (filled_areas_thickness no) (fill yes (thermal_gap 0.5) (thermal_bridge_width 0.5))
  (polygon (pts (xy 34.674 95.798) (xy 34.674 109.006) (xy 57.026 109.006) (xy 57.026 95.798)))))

